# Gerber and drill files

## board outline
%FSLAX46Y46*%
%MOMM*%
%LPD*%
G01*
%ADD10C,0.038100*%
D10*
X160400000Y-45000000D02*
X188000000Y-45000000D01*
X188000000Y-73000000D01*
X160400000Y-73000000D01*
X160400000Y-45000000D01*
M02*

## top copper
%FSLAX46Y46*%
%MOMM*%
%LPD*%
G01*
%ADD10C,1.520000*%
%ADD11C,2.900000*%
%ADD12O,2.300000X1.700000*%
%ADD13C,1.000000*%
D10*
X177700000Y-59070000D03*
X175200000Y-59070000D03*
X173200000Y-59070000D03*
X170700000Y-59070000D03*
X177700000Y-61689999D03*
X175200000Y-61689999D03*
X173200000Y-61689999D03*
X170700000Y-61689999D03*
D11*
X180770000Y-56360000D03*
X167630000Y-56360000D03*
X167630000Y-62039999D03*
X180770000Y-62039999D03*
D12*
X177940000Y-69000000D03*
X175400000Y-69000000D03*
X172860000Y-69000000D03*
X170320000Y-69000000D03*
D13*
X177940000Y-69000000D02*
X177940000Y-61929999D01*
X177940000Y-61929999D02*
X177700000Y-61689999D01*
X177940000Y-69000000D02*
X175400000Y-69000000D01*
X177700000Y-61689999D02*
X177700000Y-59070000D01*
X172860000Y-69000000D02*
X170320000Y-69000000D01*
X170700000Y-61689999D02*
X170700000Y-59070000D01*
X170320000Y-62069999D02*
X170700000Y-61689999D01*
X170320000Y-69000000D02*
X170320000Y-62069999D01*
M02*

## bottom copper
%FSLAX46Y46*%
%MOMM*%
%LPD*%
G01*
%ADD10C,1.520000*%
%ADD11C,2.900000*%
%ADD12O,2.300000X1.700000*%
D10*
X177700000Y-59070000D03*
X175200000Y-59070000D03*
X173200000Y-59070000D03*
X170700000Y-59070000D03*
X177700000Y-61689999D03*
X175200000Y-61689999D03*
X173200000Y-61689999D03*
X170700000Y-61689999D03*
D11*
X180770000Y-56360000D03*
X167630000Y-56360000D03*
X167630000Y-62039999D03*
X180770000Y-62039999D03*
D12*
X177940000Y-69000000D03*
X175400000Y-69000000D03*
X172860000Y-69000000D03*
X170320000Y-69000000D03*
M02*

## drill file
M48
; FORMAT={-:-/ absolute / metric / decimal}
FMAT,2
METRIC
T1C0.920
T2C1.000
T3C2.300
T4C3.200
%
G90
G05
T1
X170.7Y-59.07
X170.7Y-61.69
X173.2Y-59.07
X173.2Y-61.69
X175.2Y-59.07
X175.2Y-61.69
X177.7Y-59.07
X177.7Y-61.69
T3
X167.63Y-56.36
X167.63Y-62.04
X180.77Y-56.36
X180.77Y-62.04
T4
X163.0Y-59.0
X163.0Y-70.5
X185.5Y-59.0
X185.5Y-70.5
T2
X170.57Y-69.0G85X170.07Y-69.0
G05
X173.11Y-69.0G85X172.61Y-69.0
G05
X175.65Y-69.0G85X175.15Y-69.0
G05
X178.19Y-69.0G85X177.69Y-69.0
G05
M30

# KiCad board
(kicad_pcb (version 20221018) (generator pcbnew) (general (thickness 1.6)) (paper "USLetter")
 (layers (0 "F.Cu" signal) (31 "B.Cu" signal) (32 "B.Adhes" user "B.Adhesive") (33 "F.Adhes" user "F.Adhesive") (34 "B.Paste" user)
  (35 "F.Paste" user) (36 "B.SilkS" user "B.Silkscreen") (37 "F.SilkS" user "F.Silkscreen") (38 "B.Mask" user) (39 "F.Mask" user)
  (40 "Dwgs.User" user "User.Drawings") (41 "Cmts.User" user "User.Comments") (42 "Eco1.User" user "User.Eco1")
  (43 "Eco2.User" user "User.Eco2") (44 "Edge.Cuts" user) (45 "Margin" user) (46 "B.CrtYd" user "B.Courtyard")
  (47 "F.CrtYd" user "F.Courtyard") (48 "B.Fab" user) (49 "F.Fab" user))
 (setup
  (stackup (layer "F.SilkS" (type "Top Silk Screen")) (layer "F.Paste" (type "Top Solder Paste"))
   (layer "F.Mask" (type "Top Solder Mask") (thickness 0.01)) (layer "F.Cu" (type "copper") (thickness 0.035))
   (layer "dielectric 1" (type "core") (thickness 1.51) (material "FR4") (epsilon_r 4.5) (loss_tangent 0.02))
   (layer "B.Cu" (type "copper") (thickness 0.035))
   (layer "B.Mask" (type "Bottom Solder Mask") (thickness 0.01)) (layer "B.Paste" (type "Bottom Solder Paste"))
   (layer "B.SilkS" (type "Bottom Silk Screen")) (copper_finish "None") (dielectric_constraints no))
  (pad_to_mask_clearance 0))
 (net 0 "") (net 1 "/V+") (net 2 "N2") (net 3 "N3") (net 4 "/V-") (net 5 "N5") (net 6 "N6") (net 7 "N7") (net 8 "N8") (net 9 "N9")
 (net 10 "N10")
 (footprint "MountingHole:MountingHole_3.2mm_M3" (layer "F.Cu") (at 185.5 59)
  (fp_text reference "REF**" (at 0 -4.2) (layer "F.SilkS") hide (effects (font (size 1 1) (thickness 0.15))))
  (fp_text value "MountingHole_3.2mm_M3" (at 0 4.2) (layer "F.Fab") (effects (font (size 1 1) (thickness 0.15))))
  (pad "" np_thru_hole circle (at 0 0) (size 3.2 3.2) (drill 3.2) (layers "*.Cu" "*.Mask")))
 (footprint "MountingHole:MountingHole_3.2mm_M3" (layer "F.Cu") (at 185.5 70.5)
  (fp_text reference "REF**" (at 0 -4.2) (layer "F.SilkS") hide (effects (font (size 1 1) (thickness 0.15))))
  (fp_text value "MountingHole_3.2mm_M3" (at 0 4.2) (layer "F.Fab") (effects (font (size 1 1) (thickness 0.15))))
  (pad "" np_thru_hole circle (at 0 0) (size 3.2 3.2) (drill 3.2) (layers "*.Cu" "*.Mask")))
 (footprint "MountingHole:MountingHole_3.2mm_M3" (layer "F.Cu") (at 163 59)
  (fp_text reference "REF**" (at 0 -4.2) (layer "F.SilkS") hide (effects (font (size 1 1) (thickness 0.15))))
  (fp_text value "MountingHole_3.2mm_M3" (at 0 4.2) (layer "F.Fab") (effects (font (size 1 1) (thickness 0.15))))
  (pad "" np_thru_hole circle (at 0 0) (size 3.2 3.2) (drill 3.2) (layers "*.Cu" "*.Mask")))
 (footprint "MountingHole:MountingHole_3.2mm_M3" (layer "F.Cu") (at 163 70.5)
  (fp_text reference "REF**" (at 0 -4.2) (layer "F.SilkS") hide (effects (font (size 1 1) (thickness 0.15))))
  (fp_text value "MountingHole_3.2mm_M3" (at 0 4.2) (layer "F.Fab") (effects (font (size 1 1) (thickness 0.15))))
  (pad "" np_thru_hole circle (at 0 0) (size 3.2 3.2) (drill 3.2) (layers "*.Cu" "*.Mask")))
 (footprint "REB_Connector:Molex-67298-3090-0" (layer "F.Cu") (at 174.2 54.73 180)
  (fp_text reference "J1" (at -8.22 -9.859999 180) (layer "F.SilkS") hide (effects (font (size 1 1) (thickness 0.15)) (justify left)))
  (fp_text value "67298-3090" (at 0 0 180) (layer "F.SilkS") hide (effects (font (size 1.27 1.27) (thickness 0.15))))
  (pad "1" thru_hole circle (at -3.5 -4.34 180) (size 1.52 1.52) (drill 0.92) (layers "*.Cu" "*.Mask") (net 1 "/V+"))
  (pad "2" thru_hole circle (at -1 -4.34 180) (size 1.52 1.52) (drill 0.92) (layers "*.Cu" "*.Mask") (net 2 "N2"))
  (pad "3" thru_hole circle (at 1 -4.34 180) (size 1.52 1.52) (drill 0.92) (layers "*.Cu" "*.Mask") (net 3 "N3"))
  (pad "4" thru_hole circle (at 3.5 -4.34 180) (size 1.52 1.52) (drill 0.92) (layers "*.Cu" "*.Mask") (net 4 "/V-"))
  (pad "5" thru_hole circle (at -3.5 -6.959999 180) (size 1.52 1.52) (drill 0.92) (layers "*.Cu" "*.Mask") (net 1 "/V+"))
  (pad "6" thru_hole circle (at -1 -6.959999 180) (size 1.52 1.52) (drill 0.92) (layers "*.Cu" "*.Mask") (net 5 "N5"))
  (pad "7" thru_hole circle (at 1 -6.959999 180) (size 1.52 1.52) (drill 0.92) (layers "*.Cu" "*.Mask") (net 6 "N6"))
  (pad "8" thru_hole circle (at 3.5 -6.959999 180) (size 1.52 1.52) (drill 0.92) (layers "*.Cu" "*.Mask") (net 4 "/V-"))
  (pad "9" thru_hole circle (at -6.57 -1.63 180) (size 2.9 2.9) (drill 2.3) (layers "*.Cu" "*.Mask") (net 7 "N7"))
  (pad "10" thru_hole circle (at 6.57 -1.63 180) (size 2.9 2.9) (drill 2.3) (layers "*.Cu" "*.Mask") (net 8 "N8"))
  (pad "11" thru_hole circle (at 6.57 -7.309999 180) (size 2.9 2.9) (drill 2.3) (layers "*.Cu" "*.Mask") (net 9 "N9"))
  (pad "12" thru_hole circle (at -6.57 -7.309999 180) (size 2.9 2.9) (drill 2.3) (layers "*.Cu" "*.Mask") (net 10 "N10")))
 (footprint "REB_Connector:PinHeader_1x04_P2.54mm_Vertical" (layer "F.Cu") (at 174.2625 69.02)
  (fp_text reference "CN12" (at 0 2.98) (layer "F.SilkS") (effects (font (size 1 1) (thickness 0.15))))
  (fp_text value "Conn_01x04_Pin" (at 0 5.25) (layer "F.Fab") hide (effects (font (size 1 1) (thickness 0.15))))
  (pad "1" thru_hole oval (at 3.6775 -0.02 270) (size 1.7 2.3) (drill oval 1 1.5) (layers "*.Cu" "*.Mask") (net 1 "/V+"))
  (pad "2" thru_hole oval (at 1.1375 -0.02 270) (size 1.7 2.3) (drill oval 1 1.5) (layers "*.Cu" "*.Mask") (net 1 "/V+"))
  (pad "3" thru_hole oval (at -1.4025 -0.02 270) (size 1.7 2.3) (drill oval 1 1.5) (layers "*.Cu" "*.Mask") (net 4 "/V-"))
  (pad "4" thru_hole oval (at -3.9425 -0.02 270) (size 1.7 2.3) (drill oval 1 1.5) (layers "*.Cu" "*.Mask") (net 4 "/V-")))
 (gr_rect (start 160.4 45) (end 188 73) (stroke (width 0.0381) (type default)) (fill none) (layer "Edge.Cuts"))
 (segment (start 177.94 69) (end 177.94 61.929999) (width 1) (layer "F.Cu") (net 1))
 (segment (start 177.94 61.929999) (end 177.7 61.689999) (width 1) (layer "F.Cu") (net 1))
 (segment (start 177.94 69) (end 175.4 69) (width 1) (layer "F.Cu") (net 1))
 (segment (start 177.7 61.689999) (end 177.7 59.07) (width 1) (layer "F.Cu") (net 1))
 (segment (start 172.86 69) (end 170.32 69) (width 1) (layer "F.Cu") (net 4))
 (segment (start 170.7 61.689999) (end 170.7 59.07) (width 1) (layer "F.Cu") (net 4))
 (segment (start 170.32 62.069999) (end 170.7 61.689999) (width 1) (layer "F.Cu") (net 4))
 (segment (start 170.32 69) (end 170.32 62.069999) (width 1) (layer "F.Cu") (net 4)))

